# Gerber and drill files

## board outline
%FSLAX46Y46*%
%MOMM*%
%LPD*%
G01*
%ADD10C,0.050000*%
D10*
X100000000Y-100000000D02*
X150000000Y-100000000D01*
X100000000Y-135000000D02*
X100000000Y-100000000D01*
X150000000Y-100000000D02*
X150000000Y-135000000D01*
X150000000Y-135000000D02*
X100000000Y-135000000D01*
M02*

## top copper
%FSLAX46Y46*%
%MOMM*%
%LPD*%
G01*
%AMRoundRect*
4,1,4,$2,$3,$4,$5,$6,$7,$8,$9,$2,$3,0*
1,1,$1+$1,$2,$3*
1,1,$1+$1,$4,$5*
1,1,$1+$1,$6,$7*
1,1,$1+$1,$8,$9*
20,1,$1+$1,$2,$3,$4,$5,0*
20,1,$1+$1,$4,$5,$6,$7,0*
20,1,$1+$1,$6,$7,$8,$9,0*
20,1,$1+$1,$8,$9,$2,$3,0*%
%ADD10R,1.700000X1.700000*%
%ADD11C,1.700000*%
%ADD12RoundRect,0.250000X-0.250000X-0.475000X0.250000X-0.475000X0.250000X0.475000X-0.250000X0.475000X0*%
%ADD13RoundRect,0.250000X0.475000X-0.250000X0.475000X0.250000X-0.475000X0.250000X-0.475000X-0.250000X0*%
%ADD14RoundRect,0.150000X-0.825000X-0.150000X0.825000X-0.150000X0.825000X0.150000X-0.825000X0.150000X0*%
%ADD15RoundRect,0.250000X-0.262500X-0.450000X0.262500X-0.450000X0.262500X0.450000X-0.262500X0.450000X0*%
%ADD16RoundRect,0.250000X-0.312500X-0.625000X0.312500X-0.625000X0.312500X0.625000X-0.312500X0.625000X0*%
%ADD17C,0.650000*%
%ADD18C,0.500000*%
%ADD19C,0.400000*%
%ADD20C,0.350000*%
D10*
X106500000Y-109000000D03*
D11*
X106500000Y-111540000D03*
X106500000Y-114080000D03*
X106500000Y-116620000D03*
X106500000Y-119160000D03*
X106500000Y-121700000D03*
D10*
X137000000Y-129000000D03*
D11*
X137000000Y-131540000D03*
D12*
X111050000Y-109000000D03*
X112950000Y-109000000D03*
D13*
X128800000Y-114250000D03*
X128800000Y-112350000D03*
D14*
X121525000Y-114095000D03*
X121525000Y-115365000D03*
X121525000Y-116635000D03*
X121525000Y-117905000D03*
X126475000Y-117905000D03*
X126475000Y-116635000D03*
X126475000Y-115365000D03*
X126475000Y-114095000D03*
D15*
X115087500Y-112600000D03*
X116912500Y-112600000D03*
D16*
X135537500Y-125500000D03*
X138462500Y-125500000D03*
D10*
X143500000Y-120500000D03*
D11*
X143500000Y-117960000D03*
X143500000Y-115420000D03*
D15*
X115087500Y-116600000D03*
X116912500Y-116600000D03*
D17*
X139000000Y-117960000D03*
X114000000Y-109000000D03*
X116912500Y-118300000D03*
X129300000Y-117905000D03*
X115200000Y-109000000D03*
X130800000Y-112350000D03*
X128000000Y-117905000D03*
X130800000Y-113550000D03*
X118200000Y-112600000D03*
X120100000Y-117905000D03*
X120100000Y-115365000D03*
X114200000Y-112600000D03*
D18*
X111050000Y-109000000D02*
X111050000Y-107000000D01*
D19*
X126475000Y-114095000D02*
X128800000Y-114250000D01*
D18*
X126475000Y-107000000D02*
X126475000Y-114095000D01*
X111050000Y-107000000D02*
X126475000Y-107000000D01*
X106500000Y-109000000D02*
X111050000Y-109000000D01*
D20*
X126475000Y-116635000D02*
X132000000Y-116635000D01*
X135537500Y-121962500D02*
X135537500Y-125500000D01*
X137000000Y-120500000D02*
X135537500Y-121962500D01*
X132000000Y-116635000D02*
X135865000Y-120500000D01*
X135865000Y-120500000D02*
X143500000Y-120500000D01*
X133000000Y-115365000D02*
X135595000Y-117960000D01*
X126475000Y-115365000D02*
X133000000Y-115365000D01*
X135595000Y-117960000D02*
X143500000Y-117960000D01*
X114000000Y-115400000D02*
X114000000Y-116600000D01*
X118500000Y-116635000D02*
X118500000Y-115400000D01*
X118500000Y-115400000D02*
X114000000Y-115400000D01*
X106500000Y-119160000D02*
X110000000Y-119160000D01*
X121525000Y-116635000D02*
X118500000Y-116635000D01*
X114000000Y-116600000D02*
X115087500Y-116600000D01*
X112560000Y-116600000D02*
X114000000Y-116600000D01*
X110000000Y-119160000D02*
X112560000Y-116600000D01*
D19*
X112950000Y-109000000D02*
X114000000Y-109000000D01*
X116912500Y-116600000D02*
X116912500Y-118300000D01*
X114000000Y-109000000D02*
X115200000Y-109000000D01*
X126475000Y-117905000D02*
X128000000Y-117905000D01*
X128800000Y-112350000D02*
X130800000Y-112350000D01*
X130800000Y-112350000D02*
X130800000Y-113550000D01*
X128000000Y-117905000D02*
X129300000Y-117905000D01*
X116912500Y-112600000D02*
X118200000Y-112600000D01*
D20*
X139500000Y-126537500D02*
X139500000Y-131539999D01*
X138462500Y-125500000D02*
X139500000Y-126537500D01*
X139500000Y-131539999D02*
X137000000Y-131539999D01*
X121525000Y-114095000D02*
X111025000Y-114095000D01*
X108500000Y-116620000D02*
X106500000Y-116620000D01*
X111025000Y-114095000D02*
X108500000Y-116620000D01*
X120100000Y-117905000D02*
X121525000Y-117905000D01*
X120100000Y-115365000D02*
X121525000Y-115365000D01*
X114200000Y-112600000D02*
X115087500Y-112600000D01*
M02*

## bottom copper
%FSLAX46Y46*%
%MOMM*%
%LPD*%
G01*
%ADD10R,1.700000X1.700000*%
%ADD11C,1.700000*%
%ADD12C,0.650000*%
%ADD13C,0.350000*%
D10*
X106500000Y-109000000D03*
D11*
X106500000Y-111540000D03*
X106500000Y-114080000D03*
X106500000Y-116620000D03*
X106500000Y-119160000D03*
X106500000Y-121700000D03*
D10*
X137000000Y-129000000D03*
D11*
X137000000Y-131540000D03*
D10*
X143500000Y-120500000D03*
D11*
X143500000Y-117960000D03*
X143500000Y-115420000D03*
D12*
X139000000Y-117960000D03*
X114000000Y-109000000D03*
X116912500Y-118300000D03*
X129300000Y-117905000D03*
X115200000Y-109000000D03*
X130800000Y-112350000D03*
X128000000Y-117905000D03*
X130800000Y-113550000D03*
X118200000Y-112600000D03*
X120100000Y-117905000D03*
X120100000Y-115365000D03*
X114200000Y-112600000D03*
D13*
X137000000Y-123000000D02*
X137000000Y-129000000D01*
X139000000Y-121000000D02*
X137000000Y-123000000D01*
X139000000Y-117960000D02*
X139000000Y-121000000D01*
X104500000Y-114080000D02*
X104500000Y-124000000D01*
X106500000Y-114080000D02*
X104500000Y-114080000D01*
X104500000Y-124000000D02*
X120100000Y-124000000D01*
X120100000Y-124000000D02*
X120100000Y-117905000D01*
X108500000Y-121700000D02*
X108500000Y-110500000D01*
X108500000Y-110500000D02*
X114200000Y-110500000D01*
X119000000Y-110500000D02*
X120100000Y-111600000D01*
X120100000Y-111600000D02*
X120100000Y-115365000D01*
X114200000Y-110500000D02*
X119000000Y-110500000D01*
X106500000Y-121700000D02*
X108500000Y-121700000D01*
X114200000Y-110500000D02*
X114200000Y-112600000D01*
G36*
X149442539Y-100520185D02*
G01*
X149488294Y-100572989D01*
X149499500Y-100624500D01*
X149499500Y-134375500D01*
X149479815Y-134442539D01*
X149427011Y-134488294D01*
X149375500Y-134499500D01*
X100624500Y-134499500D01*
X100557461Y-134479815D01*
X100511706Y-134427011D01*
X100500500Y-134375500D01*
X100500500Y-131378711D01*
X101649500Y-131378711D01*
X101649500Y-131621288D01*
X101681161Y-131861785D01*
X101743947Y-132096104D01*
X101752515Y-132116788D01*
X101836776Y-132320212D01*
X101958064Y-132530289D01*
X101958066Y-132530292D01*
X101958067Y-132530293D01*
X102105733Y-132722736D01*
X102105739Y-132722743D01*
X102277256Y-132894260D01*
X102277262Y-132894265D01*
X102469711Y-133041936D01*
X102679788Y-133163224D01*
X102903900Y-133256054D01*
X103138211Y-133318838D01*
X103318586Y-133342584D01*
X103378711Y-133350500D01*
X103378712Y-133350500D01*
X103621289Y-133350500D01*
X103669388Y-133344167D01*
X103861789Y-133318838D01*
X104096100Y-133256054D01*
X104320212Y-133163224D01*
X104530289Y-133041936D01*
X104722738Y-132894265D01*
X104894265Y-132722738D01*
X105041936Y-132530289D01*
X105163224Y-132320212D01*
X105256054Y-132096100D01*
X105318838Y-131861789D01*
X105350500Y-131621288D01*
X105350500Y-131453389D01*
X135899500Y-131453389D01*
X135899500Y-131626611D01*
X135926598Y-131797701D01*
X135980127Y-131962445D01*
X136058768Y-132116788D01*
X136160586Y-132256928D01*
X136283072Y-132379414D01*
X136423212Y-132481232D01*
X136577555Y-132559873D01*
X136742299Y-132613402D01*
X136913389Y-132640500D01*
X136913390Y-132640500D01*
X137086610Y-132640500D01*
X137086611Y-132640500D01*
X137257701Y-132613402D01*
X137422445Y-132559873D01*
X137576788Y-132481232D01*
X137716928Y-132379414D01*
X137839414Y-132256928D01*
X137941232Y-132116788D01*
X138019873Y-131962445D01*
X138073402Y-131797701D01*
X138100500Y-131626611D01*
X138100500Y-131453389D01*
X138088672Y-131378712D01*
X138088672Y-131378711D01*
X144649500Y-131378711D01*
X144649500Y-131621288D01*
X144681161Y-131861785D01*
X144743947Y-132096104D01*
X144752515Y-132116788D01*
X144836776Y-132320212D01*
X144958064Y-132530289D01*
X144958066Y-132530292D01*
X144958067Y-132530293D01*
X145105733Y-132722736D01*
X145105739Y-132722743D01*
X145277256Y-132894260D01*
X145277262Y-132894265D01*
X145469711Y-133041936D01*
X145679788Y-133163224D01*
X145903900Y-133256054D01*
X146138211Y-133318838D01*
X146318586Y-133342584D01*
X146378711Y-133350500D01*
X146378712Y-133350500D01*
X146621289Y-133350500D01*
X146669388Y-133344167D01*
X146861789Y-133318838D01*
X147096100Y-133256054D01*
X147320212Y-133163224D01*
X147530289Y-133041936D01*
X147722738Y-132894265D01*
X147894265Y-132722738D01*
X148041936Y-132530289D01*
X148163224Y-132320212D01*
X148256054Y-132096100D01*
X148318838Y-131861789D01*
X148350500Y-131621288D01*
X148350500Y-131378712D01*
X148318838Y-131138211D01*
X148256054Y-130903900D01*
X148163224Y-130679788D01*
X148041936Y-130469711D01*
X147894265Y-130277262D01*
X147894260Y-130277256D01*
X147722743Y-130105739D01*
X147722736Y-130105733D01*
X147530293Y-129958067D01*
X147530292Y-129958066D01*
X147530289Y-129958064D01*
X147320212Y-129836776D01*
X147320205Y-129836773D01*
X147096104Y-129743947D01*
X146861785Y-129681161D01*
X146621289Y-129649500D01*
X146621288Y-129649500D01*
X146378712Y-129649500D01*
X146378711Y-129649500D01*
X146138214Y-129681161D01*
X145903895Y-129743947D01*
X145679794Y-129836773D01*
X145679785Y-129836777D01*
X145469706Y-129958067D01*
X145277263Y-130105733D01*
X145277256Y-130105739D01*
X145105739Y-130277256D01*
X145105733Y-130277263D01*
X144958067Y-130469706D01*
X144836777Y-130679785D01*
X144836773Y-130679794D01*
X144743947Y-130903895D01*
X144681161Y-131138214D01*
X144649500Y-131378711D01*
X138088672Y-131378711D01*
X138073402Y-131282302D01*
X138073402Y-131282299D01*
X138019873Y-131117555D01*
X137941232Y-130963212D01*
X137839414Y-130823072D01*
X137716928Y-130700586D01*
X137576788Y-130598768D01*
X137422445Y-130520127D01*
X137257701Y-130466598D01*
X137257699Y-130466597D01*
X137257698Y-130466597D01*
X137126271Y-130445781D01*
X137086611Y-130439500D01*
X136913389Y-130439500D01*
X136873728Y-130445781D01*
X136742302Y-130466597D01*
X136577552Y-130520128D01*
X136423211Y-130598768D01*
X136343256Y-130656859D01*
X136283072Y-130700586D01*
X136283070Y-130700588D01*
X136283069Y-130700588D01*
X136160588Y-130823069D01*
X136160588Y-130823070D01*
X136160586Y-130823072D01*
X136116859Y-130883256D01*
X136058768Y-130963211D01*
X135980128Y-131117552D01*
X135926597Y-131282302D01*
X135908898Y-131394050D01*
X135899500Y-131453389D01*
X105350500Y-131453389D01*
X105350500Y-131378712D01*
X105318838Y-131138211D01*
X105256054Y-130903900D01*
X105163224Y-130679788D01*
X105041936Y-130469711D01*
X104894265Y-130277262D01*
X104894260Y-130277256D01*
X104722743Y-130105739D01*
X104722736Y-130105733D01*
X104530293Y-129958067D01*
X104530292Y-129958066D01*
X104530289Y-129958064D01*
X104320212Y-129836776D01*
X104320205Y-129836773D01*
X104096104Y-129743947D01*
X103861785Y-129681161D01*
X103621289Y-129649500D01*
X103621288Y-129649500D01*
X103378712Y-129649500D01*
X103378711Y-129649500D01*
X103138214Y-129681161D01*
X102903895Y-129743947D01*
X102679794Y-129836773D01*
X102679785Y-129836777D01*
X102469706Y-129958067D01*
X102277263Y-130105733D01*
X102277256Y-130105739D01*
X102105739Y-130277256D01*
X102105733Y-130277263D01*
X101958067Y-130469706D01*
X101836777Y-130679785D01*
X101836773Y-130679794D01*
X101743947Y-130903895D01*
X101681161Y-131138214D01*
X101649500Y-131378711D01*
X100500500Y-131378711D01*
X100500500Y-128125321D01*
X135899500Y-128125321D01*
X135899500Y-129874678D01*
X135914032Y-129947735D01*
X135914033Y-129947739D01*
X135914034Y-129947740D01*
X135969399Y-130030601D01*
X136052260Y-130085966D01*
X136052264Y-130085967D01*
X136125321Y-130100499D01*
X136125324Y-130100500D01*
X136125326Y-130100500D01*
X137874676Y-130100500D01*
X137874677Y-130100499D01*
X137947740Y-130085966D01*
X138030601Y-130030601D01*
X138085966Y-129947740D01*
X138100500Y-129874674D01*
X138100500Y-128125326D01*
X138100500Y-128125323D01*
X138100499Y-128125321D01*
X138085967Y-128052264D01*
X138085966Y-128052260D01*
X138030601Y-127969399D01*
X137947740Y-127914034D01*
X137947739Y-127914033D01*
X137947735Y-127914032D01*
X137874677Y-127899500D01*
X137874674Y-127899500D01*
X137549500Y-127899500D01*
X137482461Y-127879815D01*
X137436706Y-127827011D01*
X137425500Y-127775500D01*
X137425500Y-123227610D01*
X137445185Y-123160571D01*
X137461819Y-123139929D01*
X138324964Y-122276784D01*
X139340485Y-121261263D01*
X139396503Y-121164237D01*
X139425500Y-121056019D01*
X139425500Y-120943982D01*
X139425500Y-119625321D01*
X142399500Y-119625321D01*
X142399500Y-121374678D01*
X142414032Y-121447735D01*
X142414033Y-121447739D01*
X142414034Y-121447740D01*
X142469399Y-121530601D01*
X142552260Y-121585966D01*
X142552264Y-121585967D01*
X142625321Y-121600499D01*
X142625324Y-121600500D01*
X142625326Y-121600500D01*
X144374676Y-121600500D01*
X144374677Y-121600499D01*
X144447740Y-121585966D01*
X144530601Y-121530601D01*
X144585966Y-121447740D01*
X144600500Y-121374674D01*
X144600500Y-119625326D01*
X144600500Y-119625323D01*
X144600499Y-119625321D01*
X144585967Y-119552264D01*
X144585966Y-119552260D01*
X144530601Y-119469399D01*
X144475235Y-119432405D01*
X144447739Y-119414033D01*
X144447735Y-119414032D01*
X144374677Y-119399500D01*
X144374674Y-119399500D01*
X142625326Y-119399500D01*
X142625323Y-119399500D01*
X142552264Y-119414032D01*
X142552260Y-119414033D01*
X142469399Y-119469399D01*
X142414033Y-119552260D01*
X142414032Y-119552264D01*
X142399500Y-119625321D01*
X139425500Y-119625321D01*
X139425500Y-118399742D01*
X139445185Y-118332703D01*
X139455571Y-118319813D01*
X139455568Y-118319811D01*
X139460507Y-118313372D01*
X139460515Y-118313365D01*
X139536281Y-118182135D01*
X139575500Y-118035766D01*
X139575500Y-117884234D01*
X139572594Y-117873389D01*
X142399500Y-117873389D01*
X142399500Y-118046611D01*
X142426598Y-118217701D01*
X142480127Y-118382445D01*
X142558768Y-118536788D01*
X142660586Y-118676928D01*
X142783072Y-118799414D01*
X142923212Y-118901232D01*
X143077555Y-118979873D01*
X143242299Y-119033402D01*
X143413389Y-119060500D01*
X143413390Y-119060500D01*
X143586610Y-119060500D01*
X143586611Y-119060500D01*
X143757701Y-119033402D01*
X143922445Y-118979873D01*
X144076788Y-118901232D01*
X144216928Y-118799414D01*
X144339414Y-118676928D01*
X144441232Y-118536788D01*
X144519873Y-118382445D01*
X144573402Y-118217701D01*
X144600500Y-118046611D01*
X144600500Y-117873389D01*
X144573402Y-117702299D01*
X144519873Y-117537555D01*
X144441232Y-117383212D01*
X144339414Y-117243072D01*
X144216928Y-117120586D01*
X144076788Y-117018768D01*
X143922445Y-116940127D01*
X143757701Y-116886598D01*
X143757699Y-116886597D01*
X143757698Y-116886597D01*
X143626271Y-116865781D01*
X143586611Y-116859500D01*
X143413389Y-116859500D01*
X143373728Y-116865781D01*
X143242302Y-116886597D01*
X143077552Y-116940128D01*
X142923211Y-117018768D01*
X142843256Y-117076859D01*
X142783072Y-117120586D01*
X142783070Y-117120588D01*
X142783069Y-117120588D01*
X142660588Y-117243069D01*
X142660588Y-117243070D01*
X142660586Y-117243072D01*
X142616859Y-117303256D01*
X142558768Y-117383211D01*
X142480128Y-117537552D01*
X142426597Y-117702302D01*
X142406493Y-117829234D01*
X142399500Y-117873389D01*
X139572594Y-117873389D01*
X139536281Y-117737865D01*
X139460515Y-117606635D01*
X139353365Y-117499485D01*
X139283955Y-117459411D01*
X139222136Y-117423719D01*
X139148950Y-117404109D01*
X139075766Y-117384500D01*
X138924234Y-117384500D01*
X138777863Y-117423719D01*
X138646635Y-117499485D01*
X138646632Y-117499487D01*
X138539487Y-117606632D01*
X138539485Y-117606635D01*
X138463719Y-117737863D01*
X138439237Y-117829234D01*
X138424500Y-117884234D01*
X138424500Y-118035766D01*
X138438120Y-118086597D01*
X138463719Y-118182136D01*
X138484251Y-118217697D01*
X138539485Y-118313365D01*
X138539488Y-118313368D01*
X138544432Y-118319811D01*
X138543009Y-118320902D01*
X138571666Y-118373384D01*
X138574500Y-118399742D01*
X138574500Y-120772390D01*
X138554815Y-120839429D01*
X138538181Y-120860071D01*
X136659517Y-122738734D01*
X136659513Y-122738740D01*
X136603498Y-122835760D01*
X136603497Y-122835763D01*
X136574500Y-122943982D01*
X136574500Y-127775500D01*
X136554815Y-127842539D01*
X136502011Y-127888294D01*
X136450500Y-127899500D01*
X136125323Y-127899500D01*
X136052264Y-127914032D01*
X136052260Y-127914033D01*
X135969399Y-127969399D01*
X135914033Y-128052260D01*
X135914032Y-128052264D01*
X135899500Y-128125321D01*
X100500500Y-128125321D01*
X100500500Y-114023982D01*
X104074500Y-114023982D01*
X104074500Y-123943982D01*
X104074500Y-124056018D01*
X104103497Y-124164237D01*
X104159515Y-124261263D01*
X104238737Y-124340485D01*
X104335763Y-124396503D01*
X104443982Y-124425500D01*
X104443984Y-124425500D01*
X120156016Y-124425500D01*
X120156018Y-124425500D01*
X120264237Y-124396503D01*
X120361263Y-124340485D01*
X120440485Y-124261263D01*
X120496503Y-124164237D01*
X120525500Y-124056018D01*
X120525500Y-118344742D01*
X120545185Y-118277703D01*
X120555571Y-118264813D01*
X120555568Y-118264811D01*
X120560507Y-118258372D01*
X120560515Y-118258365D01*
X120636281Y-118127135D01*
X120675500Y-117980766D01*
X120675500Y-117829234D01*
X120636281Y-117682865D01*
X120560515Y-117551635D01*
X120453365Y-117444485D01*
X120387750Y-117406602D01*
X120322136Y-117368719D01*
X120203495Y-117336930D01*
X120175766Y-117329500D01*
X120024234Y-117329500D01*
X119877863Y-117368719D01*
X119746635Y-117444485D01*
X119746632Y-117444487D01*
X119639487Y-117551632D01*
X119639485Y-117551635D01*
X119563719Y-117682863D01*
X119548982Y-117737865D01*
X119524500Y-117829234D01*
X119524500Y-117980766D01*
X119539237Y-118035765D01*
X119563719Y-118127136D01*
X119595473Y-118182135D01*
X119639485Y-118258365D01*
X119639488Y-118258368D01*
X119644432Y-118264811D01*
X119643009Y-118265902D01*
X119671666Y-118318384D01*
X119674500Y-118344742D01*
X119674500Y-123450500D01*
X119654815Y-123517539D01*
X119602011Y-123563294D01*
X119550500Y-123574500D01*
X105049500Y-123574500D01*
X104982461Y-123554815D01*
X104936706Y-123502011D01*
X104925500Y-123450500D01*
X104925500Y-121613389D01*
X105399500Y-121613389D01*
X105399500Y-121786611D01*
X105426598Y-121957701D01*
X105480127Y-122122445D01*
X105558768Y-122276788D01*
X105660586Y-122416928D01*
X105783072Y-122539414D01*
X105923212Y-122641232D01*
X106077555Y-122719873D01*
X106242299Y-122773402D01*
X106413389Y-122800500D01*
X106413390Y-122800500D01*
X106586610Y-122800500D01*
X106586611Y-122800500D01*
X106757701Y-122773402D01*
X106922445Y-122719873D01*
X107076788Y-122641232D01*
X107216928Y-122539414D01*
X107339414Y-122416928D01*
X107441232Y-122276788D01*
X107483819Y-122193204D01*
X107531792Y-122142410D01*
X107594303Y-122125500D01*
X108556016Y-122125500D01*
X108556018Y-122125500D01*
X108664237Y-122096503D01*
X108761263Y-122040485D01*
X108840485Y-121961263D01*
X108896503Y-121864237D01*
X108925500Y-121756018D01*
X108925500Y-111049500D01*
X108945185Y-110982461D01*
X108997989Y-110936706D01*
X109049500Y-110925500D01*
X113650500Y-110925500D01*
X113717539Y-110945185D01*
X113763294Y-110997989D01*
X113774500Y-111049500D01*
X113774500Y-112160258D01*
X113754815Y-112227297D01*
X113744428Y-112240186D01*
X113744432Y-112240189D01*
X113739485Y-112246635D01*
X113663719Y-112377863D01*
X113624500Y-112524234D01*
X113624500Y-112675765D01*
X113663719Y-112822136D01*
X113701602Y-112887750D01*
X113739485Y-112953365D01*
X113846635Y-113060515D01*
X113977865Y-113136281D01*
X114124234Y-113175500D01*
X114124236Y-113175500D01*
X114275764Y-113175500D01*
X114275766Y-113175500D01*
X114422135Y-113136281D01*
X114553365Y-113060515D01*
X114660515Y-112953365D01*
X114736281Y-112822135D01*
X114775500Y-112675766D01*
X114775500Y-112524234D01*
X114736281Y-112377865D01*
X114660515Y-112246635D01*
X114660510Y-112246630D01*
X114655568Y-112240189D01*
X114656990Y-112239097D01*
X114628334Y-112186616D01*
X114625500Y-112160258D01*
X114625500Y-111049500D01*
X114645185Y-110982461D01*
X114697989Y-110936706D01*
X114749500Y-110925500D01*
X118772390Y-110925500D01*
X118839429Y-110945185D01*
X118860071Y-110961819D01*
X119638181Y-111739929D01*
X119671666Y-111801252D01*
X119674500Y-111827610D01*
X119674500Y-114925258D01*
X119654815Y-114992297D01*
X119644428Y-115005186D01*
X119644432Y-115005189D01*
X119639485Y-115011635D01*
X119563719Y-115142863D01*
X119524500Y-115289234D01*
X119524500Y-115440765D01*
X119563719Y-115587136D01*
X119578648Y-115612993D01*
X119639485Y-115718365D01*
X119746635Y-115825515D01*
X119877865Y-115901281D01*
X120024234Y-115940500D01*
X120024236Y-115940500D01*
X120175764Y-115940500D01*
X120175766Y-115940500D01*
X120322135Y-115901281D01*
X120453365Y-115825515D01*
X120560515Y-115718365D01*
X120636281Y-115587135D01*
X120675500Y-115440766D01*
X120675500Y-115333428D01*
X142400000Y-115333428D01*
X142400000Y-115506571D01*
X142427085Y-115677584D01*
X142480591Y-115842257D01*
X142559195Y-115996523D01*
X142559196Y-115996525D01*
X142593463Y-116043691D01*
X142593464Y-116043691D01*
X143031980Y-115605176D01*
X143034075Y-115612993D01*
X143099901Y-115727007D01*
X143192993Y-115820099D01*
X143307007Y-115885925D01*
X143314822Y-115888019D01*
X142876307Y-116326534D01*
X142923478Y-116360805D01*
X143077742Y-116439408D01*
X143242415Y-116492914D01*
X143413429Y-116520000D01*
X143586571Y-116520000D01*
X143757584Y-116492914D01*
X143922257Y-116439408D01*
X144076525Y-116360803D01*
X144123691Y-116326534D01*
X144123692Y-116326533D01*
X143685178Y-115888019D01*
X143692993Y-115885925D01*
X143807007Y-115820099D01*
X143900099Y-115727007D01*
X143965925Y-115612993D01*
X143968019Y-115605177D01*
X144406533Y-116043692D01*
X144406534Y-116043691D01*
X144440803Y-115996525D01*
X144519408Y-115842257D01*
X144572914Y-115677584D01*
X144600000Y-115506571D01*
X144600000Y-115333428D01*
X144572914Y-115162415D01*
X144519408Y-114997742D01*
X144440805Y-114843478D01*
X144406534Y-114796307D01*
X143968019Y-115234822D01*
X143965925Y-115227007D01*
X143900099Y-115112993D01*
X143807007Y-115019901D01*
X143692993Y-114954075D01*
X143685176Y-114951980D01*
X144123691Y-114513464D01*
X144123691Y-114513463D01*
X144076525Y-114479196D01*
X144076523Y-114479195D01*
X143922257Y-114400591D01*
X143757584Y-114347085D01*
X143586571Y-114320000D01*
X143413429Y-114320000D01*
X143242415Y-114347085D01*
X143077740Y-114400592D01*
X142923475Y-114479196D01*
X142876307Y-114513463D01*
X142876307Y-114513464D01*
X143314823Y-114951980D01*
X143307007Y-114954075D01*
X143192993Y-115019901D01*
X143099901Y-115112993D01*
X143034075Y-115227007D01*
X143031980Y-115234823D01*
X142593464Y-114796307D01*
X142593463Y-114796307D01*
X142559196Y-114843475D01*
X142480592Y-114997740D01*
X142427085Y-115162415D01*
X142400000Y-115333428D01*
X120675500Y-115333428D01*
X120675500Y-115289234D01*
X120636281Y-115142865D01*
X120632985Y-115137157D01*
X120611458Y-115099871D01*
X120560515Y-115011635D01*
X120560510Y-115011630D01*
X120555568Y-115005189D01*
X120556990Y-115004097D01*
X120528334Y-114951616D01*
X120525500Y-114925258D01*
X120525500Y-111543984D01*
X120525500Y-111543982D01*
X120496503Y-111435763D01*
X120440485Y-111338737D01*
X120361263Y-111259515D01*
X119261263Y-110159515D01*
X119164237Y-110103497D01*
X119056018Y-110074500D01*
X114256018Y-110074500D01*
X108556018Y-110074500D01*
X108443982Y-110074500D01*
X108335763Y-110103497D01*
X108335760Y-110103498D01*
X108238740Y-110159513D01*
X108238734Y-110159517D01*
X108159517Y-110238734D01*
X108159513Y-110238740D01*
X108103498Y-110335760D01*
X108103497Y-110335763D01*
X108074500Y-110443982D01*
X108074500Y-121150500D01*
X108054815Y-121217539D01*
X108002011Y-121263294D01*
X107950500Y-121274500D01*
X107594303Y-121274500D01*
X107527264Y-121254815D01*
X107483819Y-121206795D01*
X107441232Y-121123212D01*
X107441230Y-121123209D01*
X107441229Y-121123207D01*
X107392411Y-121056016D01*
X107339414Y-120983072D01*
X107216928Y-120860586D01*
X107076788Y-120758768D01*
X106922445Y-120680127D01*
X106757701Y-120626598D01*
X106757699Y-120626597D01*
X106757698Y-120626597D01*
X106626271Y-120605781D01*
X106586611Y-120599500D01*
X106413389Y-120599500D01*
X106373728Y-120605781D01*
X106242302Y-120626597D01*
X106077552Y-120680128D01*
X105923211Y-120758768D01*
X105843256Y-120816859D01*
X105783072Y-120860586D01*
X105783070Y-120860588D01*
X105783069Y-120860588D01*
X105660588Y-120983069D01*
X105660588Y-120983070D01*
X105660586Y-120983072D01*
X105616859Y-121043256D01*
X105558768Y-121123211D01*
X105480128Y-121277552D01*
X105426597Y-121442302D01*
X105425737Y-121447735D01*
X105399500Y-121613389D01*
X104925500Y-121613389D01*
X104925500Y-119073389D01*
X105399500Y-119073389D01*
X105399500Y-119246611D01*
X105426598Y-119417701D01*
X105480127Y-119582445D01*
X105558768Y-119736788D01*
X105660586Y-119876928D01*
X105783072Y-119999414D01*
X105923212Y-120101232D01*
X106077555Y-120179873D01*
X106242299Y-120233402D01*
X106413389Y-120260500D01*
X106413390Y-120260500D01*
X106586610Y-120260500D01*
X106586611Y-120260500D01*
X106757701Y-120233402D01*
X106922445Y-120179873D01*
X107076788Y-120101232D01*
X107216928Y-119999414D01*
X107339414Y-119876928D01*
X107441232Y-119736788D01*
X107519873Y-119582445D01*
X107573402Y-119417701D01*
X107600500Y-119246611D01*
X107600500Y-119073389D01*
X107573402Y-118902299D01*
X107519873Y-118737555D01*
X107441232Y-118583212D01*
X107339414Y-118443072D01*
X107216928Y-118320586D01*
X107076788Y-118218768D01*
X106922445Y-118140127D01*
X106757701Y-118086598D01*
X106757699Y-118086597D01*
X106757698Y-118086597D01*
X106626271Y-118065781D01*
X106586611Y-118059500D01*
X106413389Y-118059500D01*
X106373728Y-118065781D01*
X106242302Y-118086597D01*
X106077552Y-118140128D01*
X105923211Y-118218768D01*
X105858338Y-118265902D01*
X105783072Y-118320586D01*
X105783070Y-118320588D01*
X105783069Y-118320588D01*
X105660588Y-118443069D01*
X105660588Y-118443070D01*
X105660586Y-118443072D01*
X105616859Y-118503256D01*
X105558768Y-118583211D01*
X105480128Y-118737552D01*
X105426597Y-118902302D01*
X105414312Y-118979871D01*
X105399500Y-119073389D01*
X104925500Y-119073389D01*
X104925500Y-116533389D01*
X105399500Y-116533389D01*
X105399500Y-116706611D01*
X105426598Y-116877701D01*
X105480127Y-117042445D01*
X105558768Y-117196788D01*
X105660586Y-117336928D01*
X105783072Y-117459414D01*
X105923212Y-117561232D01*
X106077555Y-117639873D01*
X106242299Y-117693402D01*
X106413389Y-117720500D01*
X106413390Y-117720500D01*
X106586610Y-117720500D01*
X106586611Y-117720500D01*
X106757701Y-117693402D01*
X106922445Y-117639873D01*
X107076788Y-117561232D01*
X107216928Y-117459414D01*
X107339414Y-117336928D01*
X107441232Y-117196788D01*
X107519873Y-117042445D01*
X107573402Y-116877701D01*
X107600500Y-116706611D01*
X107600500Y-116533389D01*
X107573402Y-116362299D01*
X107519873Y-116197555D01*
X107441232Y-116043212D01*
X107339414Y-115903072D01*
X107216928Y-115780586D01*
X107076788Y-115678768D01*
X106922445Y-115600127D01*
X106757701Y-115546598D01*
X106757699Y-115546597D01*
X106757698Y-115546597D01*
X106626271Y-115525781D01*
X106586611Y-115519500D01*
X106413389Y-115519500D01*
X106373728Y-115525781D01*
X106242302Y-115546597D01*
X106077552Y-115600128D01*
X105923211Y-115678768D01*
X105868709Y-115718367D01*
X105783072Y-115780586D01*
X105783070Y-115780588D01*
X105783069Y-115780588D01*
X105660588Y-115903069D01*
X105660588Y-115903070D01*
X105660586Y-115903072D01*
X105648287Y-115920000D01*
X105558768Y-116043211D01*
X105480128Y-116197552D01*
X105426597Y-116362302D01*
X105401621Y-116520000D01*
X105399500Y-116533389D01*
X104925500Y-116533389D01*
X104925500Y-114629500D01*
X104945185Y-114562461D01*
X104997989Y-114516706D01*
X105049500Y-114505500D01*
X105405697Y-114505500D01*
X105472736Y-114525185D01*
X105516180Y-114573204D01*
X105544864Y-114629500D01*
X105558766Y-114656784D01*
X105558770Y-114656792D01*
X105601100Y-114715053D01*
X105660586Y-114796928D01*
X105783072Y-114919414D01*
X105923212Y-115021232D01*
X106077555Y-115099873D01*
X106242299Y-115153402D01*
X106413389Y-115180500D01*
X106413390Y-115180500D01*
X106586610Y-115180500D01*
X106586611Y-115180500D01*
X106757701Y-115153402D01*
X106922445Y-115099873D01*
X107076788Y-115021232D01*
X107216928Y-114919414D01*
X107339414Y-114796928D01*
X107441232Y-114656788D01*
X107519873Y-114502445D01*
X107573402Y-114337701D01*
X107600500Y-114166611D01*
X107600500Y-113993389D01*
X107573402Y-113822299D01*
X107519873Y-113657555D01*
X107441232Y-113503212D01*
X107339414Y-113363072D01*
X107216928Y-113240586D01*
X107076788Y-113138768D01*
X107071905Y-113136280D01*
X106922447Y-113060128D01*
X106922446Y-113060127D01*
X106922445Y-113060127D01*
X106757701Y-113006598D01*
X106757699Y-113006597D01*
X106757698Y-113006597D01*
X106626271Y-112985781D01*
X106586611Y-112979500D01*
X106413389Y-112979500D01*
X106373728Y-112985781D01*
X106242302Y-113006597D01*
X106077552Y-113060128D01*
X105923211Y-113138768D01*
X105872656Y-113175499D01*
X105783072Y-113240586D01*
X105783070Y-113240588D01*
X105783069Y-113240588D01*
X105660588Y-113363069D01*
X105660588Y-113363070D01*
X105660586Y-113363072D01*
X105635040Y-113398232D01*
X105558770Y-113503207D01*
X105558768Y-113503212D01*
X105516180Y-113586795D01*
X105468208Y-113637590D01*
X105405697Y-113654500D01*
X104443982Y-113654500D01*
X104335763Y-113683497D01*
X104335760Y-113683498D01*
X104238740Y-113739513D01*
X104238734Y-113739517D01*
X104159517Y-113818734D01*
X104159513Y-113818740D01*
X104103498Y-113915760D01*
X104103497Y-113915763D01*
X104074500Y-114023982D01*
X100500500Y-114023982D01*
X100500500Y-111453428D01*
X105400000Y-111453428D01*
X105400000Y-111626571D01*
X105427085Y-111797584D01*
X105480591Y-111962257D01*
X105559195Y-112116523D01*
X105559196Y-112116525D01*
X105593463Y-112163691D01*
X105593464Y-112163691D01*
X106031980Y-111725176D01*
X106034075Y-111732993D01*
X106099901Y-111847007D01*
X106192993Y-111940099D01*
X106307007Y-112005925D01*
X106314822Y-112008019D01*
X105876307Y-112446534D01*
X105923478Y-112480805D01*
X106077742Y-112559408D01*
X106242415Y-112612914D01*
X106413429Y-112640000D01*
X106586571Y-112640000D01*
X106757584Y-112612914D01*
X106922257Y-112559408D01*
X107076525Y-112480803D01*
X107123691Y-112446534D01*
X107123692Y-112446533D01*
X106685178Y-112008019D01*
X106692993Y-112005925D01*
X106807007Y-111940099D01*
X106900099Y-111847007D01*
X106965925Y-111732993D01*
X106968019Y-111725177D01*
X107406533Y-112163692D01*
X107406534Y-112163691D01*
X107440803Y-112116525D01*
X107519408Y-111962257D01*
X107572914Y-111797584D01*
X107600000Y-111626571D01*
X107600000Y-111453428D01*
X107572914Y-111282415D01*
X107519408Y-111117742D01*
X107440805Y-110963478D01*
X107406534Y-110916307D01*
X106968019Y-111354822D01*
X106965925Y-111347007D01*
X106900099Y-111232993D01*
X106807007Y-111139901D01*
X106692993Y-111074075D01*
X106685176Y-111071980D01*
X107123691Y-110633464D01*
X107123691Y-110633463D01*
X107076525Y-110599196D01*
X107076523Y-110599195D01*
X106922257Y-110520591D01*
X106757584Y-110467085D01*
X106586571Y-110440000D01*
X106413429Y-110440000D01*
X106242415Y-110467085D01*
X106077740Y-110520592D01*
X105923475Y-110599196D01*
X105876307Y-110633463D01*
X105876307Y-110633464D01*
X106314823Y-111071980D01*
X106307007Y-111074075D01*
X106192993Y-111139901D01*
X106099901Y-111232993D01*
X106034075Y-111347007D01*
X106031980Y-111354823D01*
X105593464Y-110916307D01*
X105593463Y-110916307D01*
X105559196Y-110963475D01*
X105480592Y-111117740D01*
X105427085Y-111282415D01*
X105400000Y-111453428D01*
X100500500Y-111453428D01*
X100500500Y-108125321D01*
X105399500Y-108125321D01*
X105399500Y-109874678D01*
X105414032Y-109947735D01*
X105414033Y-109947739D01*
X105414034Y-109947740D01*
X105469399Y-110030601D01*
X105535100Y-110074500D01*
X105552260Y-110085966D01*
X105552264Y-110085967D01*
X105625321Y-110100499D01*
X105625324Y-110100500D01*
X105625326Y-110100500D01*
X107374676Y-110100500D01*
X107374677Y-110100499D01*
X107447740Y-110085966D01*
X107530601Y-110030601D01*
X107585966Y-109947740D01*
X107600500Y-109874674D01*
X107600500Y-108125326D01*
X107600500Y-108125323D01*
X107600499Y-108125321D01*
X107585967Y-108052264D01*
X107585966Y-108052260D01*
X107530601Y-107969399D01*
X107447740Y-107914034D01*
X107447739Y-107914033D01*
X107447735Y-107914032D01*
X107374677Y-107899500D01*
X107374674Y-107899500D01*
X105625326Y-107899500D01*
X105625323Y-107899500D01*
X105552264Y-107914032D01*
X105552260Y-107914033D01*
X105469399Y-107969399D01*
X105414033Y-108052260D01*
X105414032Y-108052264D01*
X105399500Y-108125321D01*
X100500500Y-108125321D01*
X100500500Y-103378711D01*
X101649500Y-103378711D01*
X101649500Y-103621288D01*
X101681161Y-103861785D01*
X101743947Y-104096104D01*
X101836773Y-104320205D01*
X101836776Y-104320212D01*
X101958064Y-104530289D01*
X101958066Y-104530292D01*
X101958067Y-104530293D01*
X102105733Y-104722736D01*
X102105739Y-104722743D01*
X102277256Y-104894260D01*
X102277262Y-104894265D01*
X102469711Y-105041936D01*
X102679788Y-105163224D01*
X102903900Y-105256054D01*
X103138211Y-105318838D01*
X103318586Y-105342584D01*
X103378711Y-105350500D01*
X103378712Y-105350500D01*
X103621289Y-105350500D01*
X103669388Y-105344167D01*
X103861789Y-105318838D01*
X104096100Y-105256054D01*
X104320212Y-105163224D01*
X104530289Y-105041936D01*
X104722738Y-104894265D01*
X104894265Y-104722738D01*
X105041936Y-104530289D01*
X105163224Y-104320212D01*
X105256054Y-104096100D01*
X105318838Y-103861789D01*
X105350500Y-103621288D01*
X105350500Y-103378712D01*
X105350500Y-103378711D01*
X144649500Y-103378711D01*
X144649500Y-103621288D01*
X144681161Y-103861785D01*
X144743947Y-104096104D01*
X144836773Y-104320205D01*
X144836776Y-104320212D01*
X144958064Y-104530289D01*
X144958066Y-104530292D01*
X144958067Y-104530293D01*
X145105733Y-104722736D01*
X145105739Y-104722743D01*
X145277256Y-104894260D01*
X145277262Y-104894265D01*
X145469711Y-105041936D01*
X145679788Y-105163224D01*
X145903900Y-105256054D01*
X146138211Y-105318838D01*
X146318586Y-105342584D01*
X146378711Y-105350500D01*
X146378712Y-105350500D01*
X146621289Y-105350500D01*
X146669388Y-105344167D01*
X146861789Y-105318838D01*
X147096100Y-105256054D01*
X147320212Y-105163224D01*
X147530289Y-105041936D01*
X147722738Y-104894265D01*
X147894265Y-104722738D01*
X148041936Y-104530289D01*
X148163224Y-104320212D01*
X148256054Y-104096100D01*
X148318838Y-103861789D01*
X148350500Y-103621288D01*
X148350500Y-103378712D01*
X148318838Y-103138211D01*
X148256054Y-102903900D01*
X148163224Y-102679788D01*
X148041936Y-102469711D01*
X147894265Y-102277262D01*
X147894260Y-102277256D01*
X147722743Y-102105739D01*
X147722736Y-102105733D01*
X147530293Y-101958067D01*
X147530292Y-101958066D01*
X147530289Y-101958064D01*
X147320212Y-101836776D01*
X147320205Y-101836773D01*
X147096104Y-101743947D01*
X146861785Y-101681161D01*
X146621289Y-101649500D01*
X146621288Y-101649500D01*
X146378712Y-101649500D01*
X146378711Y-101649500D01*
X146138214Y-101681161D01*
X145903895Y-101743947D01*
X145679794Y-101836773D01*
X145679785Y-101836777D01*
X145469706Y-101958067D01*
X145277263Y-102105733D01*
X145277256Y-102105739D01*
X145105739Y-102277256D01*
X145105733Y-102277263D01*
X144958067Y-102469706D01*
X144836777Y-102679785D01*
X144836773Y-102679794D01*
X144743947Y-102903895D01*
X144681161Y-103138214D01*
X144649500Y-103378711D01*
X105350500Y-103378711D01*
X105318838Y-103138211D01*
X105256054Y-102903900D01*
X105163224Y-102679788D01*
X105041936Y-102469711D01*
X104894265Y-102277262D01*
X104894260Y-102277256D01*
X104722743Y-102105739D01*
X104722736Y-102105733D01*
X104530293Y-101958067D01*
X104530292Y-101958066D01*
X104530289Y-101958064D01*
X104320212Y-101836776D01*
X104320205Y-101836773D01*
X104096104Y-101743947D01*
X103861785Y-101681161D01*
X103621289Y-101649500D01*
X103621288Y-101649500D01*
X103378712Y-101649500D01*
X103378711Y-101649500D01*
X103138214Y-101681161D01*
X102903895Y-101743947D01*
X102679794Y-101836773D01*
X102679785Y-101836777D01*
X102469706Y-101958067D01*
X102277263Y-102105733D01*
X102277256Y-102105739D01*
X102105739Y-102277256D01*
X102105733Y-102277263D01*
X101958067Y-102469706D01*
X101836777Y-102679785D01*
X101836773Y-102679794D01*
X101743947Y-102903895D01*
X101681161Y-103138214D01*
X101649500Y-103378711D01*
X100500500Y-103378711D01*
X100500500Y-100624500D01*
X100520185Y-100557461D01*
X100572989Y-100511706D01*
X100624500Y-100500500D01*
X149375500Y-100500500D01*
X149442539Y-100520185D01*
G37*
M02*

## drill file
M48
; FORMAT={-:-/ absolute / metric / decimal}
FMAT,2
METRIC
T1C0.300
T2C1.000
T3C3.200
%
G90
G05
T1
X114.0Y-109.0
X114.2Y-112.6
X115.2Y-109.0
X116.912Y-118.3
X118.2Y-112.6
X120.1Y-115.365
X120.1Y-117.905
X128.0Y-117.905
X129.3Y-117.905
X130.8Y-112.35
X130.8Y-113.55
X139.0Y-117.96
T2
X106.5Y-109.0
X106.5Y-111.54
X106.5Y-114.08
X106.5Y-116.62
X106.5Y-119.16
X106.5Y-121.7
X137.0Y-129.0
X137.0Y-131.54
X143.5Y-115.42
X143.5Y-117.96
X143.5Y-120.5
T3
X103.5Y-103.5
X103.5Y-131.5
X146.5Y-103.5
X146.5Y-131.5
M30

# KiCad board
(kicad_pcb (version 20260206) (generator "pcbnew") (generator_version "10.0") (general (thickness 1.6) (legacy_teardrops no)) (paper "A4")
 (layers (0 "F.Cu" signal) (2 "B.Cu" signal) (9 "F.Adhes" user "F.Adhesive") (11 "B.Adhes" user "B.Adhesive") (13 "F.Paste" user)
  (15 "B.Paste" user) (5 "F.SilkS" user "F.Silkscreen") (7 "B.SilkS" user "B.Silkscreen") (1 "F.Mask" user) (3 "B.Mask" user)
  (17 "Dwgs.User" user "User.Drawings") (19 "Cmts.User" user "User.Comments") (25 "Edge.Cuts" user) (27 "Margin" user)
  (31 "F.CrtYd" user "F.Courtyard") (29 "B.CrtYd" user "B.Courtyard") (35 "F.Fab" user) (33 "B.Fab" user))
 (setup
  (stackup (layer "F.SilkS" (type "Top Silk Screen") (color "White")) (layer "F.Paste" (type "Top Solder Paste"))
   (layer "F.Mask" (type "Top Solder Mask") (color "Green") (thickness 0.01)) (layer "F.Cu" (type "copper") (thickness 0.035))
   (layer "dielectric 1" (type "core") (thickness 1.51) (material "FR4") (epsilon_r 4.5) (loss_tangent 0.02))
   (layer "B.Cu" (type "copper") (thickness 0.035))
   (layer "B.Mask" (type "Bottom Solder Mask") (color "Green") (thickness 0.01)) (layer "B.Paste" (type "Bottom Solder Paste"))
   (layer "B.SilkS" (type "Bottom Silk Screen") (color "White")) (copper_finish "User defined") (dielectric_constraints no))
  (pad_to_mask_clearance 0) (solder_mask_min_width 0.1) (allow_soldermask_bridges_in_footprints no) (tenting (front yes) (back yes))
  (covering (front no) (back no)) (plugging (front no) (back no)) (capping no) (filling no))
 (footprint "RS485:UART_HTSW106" (layer "F.Cu") (at 106.5 109)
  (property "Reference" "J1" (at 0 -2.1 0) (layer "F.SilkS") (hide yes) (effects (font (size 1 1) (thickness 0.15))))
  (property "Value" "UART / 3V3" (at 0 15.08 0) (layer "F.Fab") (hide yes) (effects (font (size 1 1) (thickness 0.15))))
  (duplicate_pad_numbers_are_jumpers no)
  (pad "1" thru_hole rect (at 0 0) (size 1.7 1.7) (drill 1) (layers "*.Cu" "*.Mask") (remove_unused_layers no) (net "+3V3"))
  (pad "2" thru_hole circle (at 0 2.54) (size 1.7 1.7) (drill 1) (layers "*.Cu" "*.Mask") (remove_unused_layers no) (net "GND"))
  (pad "3" thru_hole circle (at 0 5.08) (size 1.7 1.7) (drill 1) (layers "*.Cu" "*.Mask") (remove_unused_layers no) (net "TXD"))
  (pad "4" thru_hole circle (at 0 7.62) (size 1.7 1.7) (drill 1) (layers "*.Cu" "*.Mask") (remove_unused_layers no) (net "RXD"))
  (pad "5" thru_hole circle (at 0 10.16) (size 1.7 1.7) (drill 1) (layers "*.Cu" "*.Mask") (remove_unused_layers no) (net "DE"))
  (pad "6" thru_hole circle (at 0 12.7) (size 1.7 1.7) (drill 1) (layers "*.Cu" "*.Mask") (remove_unused_layers no) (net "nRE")))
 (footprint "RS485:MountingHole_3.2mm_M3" (layer "F.Cu") (at 103.5 103.5)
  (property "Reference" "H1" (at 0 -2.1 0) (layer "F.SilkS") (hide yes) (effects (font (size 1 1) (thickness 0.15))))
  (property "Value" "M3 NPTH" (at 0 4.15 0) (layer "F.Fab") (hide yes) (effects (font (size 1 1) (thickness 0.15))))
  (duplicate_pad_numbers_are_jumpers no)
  (pad "" np_thru_hole circle (at 0 0) (size 3.2 3.2) (drill 3.2) (layers "*.Cu" "*.Mask")))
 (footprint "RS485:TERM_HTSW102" (layer "F.Cu") (at 137 129)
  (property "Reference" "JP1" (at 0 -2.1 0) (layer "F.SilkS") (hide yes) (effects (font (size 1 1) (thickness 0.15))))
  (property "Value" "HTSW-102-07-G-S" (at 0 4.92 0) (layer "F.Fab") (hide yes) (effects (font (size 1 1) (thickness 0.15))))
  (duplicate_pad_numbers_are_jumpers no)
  (pad "1" thru_hole rect (at 0 0) (size 1.7 1.7) (drill 1) (layers "*.Cu" "*.Mask") (remove_unused_layers no) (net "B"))
  (pad "2" thru_hole circle (at 0 2.54) (size 1.7 1.7) (drill 1) (layers "*.Cu" "*.Mask") (remove_unused_layers no) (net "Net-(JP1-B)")))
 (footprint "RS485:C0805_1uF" (layer "F.Cu") (at 112 109)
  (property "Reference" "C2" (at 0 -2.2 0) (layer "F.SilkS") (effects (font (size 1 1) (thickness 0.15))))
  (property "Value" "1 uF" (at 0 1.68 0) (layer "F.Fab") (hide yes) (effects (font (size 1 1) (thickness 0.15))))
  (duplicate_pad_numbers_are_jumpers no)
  (pad "1" smd roundrect (at -0.95 0) (size 1 1.45) (layers "F.Cu" "F.Mask" "F.Paste") (roundrect_rratio 0.25) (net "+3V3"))
  (pad "2" smd roundrect (at 0.95 0) (size 1 1.45) (layers "F.Cu" "F.Mask" "F.Paste") (roundrect_rratio 0.25) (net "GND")))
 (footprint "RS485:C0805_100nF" (layer "F.Cu") (at 128.8 113.3 90)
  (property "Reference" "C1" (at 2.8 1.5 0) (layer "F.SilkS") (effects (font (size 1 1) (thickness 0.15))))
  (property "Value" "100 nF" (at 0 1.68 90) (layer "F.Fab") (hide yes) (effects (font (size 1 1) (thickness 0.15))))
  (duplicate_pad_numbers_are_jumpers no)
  (pad "1" smd roundrect (at -0.95 0 90) (size 1 1.45) (layers "F.Cu" "F.Mask" "F.Paste") (roundrect_rratio 0.25) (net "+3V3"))
  (pad "2" smd roundrect (at 0.95 0 90) (size 1 1.45) (layers "F.Cu" "F.Mask" "F.Paste") (roundrect_rratio 0.25) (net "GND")))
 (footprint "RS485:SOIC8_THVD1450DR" (layer "F.Cu") (at 124 116)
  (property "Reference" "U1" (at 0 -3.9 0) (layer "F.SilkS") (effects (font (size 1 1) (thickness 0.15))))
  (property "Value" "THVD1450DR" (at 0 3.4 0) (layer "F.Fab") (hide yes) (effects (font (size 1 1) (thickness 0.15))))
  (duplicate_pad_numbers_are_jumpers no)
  (pad "1" smd roundrect (at -2.475 -1.905) (size 1.95 0.6) (layers "F.Cu" "F.Mask" "F.Paste") (roundrect_rratio 0.25) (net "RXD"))
  (pad "2" smd roundrect (at -2.475 -0.635) (size 1.95 0.6) (layers "F.Cu" "F.Mask" "F.Paste") (roundrect_rratio 0.25) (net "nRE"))
  (pad "3" smd roundrect (at -2.475 0.635) (size 1.95 0.6) (layers "F.Cu" "F.Mask" "F.Paste") (roundrect_rratio 0.25) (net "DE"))
  (pad "4" smd roundrect (at -2.475 1.905) (size 1.95 0.6) (layers "F.Cu" "F.Mask" "F.Paste") (roundrect_rratio 0.25) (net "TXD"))
  (pad "5" smd roundrect (at 2.475 1.905) (size 1.95 0.6) (layers "F.Cu" "F.Mask" "F.Paste") (roundrect_rratio 0.25) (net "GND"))
  (pad "6" smd roundrect (at 2.475 0.635) (size 1.95 0.6) (layers "F.Cu" "F.Mask" "F.Paste") (roundrect_rratio 0.25) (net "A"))
  (pad "7" smd roundrect (at 2.475 -0.635) (size 1.95 0.6) (layers "F.Cu" "F.Mask" "F.Paste") (roundrect_rratio 0.25) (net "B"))
  (pad "8" smd roundrect (at 2.475 -1.905) (size 1.95 0.6) (layers "F.Cu" "F.Mask" "F.Paste") (roundrect_rratio 0.25) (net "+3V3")))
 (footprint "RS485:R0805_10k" (layer "F.Cu") (at 116 112.6)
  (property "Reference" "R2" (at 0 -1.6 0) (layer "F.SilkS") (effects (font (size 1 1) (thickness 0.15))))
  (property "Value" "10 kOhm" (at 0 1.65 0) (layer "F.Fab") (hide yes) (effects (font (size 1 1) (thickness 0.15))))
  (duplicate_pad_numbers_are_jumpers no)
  (pad "1" smd roundrect (at -0.9125 0) (size 1.025 1.4) (layers "F.Cu" "F.Mask" "F.Paste") (roundrect_rratio 0.243902) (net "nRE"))
  (pad "2" smd roundrect (at 0.9125 0) (size 1.025 1.4) (layers "F.Cu" "F.Mask" "F.Paste") (roundrect_rratio 0.243902) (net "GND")))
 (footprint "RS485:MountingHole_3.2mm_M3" (layer "F.Cu") (at 103.5 131.5)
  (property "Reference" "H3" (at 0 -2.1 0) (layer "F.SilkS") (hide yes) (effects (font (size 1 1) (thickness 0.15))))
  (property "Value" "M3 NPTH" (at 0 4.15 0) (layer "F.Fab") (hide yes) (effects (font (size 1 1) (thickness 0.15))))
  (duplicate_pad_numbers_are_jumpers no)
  (pad "" np_thru_hole circle (at 0 0) (size 3.2 3.2) (drill 3.2) (layers "*.Cu" "*.Mask")))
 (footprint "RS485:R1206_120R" (layer "F.Cu") (at 137 125.5)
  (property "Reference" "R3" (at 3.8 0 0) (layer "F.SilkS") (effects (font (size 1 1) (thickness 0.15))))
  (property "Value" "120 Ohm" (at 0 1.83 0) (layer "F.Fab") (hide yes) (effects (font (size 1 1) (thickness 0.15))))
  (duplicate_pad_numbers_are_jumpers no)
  (pad "1" smd roundrect (at -1.4625 0) (size 1.125 1.75) (layers "F.Cu" "F.Mask" "F.Paste") (roundrect_rratio 0.222222) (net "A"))
  (pad "2" smd roundrect (at 1.4625 0) (size 1.125 1.75) (layers "F.Cu" "F.Mask" "F.Paste") (roundrect_rratio 0.222222) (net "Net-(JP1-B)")))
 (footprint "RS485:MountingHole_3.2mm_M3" (layer "F.Cu") (at 146.5 103.5)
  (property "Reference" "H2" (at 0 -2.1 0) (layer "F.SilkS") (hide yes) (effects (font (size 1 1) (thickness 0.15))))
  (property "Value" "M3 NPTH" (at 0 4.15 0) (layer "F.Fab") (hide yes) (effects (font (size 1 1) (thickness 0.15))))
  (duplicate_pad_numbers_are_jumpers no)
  (pad "" np_thru_hole circle (at 0 0) (size 3.2 3.2) (drill 3.2) (layers "*.Cu" "*.Mask")))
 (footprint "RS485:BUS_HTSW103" (layer "F.Cu") (at 143.5 120.5 180)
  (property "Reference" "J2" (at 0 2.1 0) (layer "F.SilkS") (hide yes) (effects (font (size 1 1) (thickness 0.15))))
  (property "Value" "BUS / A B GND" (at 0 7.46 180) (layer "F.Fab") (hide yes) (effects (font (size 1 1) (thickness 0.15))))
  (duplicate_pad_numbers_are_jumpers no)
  (pad "1" thru_hole rect (at 0 0 180) (size 1.7 1.7) (drill 1) (layers "*.Cu" "*.Mask") (remove_unused_layers no) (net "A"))
  (pad "2" thru_hole circle (at 0 2.54 180) (size 1.7 1.7) (drill 1) (layers "*.Cu" "*.Mask") (remove_unused_layers no) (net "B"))
  (pad "3" thru_hole circle (at 0 5.08 180) (size 1.7 1.7) (drill 1) (layers "*.Cu" "*.Mask") (remove_unused_layers no) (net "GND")))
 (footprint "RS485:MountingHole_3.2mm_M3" (layer "F.Cu") (at 146.5 131.5)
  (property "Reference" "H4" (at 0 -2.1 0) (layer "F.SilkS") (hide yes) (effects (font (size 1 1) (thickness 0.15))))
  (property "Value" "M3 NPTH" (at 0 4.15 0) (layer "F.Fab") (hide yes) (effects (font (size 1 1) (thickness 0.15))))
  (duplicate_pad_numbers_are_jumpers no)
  (pad "" np_thru_hole circle (at 0 0) (size 3.2 3.2) (drill 3.2) (layers "*.Cu" "*.Mask")))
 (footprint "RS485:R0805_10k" (layer "F.Cu") (at 116 116.6)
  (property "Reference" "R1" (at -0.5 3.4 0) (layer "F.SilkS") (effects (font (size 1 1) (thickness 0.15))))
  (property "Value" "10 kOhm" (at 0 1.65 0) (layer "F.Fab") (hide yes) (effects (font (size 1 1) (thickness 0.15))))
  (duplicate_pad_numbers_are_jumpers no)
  (pad "1" smd roundrect (at -0.9125 0) (size 1.025 1.4) (layers "F.Cu" "F.Mask" "F.Paste") (roundrect_rratio 0.243902) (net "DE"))
  (pad "2" smd roundrect (at 0.9125 0) (size 1.025 1.4) (layers "F.Cu" "F.Mask" "F.Paste") (roundrect_rratio 0.243902) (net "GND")))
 (gr_line (start 100 100) (end 150 100) (stroke (width 0.05) (type default)) (layer "Edge.Cuts"))
 (gr_line (start 100 135) (end 100 100) (stroke (width 0.05) (type default)) (layer "Edge.Cuts"))
 (gr_line (start 150 100) (end 150 135) (stroke (width 0.05) (type default)) (layer "Edge.Cuts"))
 (gr_line (start 150 135) (end 100 135) (stroke (width 0.05) (type default)) (layer "Edge.Cuts"))
 (segment (start 111.05 109) (end 111.05 107) (width 0.5) (layer "F.Cu") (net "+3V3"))
 (segment (start 126.475 114.095) (end 128.8 114.25) (width 0.4) (layer "F.Cu") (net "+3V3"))
 (segment (start 126.475 107) (end 126.475 114.095) (width 0.5) (layer "F.Cu") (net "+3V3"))
 (segment (start 111.05 107) (end 126.475 107) (width 0.5) (layer "F.Cu") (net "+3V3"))
 (segment (start 106.5 109) (end 111.05 109) (width 0.5) (layer "F.Cu") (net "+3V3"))
 (segment (start 126.475 116.635) (end 132 116.635) (width 0.35) (layer "F.Cu") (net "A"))
 (segment (start 135.5375 121.9625) (end 135.5375 125.5) (width 0.35) (layer "F.Cu") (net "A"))
 (segment (start 137 120.5) (end 135.5375 121.9625) (width 0.35) (layer "F.Cu") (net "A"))
 (segment (start 132 116.635) (end 135.865 120.5) (width 0.35) (layer "F.Cu") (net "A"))
 (segment (start 135.865 120.5) (end 143.5 120.5) (width 0.35) (layer "F.Cu") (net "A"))
 (segment (start 133 115.365) (end 135.595 117.96) (width 0.35) (layer "F.Cu") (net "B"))
 (segment (start 126.475 115.365) (end 133 115.365) (width 0.35) (layer "F.Cu") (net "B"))
 (segment (start 135.595 117.96) (end 143.5 117.96) (width 0.35) (layer "F.Cu") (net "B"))
 (via (at 139 117.96) (size 0.65) (drill 0.3) (layers "F.Cu" "B.Cu") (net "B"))
 (segment (start 137 123) (end 137 129) (width 0.35) (layer "B.Cu") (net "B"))
 (segment (start 139 121) (end 137 123) (width 0.35) (layer "B.Cu") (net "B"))
 (segment (start 139 117.96) (end 139 121) (width 0.35) (layer "B.Cu") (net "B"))
 (segment (start 114 115.4) (end 114 116.6) (width 0.35) (layer "F.Cu") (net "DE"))
 (segment (start 118.5 116.635) (end 118.5 115.4) (width 0.35) (layer "F.Cu") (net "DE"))
 (segment (start 118.5 115.4) (end 114 115.4) (width 0.35) (layer "F.Cu") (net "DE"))
 (segment (start 106.5 119.16) (end 110 119.16) (width 0.35) (layer "F.Cu") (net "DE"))
 (segment (start 121.525 116.635) (end 118.5 116.635) (width 0.35) (layer "F.Cu") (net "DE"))
 (segment (start 114 116.6) (end 115.0875 116.6) (width 0.35) (layer "F.Cu") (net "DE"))
 (segment (start 112.56 116.6) (end 114 116.6) (width 0.35) (layer "F.Cu") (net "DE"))
 (segment (start 110 119.16) (end 112.56 116.6) (width 0.35) (layer "F.Cu") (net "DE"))
 (segment (start 112.95 109) (end 114 109) (width 0.4) (layer "F.Cu") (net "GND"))
 (segment (start 116.9125 116.6) (end 116.9125 118.3) (width 0.4) (layer "F.Cu") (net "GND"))
 (segment (start 114 109) (end 115.2 109) (width 0.4) (layer "F.Cu") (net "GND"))
 (segment (start 126.475 117.905) (end 128 117.905) (width 0.4) (layer "F.Cu") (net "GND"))
 (segment (start 128.8 112.35) (end 130.8 112.35) (width 0.4) (layer "F.Cu") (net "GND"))
 (segment (start 130.8 112.35) (end 130.8 113.55) (width 0.4) (layer "F.Cu") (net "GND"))
 (segment (start 128 117.905) (end 129.3 117.905) (width 0.4) (layer "F.Cu") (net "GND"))
 (segment (start 116.9125 112.6) (end 118.2 112.6) (width 0.4) (layer "F.Cu") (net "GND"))
 (via (at 114 109) (size 0.65) (drill 0.3) (layers "F.Cu" "B.Cu") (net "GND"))
 (via (at 116.9125 118.3) (size 0.65) (drill 0.3) (layers "F.Cu" "B.Cu") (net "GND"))
 (via (at 129.3 117.905) (size 0.65) (drill 0.3) (layers "F.Cu" "B.Cu") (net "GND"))
 (via (at 115.2 109) (size 0.65) (drill 0.3) (layers "F.Cu" "B.Cu") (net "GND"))
 (via (at 130.8 112.35) (size 0.65) (drill 0.3) (layers "F.Cu" "B.Cu") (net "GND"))
 (via (at 128 117.905) (size 0.65) (drill 0.3) (layers "F.Cu" "B.Cu") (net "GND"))
 (via (at 130.8 113.55) (size 0.65) (drill 0.3) (layers "F.Cu" "B.Cu") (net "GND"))
 (via (at 118.2 112.6) (size 0.65) (drill 0.3) (layers "F.Cu" "B.Cu") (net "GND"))
 (segment (start 139.5 126.5375) (end 139.5 131.539999) (width 0.35) (layer "F.Cu") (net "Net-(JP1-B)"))
 (segment (start 138.4625 125.5) (end 139.5 126.5375) (width 0.35) (layer "F.Cu") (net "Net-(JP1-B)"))
 (segment (start 139.5 131.539999) (end 137 131.539999) (width 0.35) (layer "F.Cu") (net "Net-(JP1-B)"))
 (segment (start 121.525 114.095) (end 111.025 114.095) (width 0.35) (layer "F.Cu") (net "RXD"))
 (segment (start 108.5 116.62) (end 106.5 116.62) (width 0.35) (layer "F.Cu") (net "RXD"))
 (segment (start 111.025 114.095) (end 108.5 116.62) (width 0.35) (layer "F.Cu") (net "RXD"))
 (segment (start 120.1 117.905) (end 121.525 117.905) (width 0.35) (layer "F.Cu") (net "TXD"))
 (via (at 120.1 117.905) (size 0.65) (drill 0.3) (layers "F.Cu" "B.Cu") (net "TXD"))
 (segment (start 104.5 114.08) (end 104.5 124) (width 0.35) (layer "B.Cu") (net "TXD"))
 (segment (start 106.5 114.08) (end 104.5 114.08) (width 0.35) (layer "B.Cu") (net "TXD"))
 (segment (start 104.5 124) (end 120.1 124) (width 0.35) (layer "B.Cu") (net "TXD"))
 (segment (start 120.1 124) (end 120.1 117.905) (width 0.35) (layer "B.Cu") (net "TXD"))
 (segment (start 120.1 115.365) (end 121.525 115.365) (width 0.35) (layer "F.Cu") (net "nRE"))
 (segment (start 114.2 112.6) (end 115.0875 112.6) (width 0.35) (layer "F.Cu") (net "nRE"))
 (via (at 120.1 115.365) (size 0.65) (drill 0.3) (layers "F.Cu" "B.Cu") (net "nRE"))
 (via (at 114.2 112.6) (size 0.65) (drill 0.3) (layers "F.Cu" "B.Cu") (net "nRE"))
 (segment (start 108.5 121.7) (end 108.5 110.5) (width 0.35) (layer "B.Cu") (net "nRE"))
 (segment (start 108.5 110.5) (end 114.2 110.5) (width 0.35) (layer "B.Cu") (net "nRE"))
 (segment (start 119 110.5) (end 120.1 111.6) (width 0.35) (layer "B.Cu") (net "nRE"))
 (segment (start 120.1 111.6) (end 120.1 115.365) (width 0.35) (layer "B.Cu") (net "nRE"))
 (segment (start 114.2 110.5) (end 119 110.5) (width 0.35) (layer "B.Cu") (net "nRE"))
 (segment (start 106.5 121.7) (end 108.5 121.7) (width 0.35) (layer "B.Cu") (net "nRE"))
 (segment (start 114.2 110.5) (end 114.2 112.6) (width 0.35) (layer "B.Cu") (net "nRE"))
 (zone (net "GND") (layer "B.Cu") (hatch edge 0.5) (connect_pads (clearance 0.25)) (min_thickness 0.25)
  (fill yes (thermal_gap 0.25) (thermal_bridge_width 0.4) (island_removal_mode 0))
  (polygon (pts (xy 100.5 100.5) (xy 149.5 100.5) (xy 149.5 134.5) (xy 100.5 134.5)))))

